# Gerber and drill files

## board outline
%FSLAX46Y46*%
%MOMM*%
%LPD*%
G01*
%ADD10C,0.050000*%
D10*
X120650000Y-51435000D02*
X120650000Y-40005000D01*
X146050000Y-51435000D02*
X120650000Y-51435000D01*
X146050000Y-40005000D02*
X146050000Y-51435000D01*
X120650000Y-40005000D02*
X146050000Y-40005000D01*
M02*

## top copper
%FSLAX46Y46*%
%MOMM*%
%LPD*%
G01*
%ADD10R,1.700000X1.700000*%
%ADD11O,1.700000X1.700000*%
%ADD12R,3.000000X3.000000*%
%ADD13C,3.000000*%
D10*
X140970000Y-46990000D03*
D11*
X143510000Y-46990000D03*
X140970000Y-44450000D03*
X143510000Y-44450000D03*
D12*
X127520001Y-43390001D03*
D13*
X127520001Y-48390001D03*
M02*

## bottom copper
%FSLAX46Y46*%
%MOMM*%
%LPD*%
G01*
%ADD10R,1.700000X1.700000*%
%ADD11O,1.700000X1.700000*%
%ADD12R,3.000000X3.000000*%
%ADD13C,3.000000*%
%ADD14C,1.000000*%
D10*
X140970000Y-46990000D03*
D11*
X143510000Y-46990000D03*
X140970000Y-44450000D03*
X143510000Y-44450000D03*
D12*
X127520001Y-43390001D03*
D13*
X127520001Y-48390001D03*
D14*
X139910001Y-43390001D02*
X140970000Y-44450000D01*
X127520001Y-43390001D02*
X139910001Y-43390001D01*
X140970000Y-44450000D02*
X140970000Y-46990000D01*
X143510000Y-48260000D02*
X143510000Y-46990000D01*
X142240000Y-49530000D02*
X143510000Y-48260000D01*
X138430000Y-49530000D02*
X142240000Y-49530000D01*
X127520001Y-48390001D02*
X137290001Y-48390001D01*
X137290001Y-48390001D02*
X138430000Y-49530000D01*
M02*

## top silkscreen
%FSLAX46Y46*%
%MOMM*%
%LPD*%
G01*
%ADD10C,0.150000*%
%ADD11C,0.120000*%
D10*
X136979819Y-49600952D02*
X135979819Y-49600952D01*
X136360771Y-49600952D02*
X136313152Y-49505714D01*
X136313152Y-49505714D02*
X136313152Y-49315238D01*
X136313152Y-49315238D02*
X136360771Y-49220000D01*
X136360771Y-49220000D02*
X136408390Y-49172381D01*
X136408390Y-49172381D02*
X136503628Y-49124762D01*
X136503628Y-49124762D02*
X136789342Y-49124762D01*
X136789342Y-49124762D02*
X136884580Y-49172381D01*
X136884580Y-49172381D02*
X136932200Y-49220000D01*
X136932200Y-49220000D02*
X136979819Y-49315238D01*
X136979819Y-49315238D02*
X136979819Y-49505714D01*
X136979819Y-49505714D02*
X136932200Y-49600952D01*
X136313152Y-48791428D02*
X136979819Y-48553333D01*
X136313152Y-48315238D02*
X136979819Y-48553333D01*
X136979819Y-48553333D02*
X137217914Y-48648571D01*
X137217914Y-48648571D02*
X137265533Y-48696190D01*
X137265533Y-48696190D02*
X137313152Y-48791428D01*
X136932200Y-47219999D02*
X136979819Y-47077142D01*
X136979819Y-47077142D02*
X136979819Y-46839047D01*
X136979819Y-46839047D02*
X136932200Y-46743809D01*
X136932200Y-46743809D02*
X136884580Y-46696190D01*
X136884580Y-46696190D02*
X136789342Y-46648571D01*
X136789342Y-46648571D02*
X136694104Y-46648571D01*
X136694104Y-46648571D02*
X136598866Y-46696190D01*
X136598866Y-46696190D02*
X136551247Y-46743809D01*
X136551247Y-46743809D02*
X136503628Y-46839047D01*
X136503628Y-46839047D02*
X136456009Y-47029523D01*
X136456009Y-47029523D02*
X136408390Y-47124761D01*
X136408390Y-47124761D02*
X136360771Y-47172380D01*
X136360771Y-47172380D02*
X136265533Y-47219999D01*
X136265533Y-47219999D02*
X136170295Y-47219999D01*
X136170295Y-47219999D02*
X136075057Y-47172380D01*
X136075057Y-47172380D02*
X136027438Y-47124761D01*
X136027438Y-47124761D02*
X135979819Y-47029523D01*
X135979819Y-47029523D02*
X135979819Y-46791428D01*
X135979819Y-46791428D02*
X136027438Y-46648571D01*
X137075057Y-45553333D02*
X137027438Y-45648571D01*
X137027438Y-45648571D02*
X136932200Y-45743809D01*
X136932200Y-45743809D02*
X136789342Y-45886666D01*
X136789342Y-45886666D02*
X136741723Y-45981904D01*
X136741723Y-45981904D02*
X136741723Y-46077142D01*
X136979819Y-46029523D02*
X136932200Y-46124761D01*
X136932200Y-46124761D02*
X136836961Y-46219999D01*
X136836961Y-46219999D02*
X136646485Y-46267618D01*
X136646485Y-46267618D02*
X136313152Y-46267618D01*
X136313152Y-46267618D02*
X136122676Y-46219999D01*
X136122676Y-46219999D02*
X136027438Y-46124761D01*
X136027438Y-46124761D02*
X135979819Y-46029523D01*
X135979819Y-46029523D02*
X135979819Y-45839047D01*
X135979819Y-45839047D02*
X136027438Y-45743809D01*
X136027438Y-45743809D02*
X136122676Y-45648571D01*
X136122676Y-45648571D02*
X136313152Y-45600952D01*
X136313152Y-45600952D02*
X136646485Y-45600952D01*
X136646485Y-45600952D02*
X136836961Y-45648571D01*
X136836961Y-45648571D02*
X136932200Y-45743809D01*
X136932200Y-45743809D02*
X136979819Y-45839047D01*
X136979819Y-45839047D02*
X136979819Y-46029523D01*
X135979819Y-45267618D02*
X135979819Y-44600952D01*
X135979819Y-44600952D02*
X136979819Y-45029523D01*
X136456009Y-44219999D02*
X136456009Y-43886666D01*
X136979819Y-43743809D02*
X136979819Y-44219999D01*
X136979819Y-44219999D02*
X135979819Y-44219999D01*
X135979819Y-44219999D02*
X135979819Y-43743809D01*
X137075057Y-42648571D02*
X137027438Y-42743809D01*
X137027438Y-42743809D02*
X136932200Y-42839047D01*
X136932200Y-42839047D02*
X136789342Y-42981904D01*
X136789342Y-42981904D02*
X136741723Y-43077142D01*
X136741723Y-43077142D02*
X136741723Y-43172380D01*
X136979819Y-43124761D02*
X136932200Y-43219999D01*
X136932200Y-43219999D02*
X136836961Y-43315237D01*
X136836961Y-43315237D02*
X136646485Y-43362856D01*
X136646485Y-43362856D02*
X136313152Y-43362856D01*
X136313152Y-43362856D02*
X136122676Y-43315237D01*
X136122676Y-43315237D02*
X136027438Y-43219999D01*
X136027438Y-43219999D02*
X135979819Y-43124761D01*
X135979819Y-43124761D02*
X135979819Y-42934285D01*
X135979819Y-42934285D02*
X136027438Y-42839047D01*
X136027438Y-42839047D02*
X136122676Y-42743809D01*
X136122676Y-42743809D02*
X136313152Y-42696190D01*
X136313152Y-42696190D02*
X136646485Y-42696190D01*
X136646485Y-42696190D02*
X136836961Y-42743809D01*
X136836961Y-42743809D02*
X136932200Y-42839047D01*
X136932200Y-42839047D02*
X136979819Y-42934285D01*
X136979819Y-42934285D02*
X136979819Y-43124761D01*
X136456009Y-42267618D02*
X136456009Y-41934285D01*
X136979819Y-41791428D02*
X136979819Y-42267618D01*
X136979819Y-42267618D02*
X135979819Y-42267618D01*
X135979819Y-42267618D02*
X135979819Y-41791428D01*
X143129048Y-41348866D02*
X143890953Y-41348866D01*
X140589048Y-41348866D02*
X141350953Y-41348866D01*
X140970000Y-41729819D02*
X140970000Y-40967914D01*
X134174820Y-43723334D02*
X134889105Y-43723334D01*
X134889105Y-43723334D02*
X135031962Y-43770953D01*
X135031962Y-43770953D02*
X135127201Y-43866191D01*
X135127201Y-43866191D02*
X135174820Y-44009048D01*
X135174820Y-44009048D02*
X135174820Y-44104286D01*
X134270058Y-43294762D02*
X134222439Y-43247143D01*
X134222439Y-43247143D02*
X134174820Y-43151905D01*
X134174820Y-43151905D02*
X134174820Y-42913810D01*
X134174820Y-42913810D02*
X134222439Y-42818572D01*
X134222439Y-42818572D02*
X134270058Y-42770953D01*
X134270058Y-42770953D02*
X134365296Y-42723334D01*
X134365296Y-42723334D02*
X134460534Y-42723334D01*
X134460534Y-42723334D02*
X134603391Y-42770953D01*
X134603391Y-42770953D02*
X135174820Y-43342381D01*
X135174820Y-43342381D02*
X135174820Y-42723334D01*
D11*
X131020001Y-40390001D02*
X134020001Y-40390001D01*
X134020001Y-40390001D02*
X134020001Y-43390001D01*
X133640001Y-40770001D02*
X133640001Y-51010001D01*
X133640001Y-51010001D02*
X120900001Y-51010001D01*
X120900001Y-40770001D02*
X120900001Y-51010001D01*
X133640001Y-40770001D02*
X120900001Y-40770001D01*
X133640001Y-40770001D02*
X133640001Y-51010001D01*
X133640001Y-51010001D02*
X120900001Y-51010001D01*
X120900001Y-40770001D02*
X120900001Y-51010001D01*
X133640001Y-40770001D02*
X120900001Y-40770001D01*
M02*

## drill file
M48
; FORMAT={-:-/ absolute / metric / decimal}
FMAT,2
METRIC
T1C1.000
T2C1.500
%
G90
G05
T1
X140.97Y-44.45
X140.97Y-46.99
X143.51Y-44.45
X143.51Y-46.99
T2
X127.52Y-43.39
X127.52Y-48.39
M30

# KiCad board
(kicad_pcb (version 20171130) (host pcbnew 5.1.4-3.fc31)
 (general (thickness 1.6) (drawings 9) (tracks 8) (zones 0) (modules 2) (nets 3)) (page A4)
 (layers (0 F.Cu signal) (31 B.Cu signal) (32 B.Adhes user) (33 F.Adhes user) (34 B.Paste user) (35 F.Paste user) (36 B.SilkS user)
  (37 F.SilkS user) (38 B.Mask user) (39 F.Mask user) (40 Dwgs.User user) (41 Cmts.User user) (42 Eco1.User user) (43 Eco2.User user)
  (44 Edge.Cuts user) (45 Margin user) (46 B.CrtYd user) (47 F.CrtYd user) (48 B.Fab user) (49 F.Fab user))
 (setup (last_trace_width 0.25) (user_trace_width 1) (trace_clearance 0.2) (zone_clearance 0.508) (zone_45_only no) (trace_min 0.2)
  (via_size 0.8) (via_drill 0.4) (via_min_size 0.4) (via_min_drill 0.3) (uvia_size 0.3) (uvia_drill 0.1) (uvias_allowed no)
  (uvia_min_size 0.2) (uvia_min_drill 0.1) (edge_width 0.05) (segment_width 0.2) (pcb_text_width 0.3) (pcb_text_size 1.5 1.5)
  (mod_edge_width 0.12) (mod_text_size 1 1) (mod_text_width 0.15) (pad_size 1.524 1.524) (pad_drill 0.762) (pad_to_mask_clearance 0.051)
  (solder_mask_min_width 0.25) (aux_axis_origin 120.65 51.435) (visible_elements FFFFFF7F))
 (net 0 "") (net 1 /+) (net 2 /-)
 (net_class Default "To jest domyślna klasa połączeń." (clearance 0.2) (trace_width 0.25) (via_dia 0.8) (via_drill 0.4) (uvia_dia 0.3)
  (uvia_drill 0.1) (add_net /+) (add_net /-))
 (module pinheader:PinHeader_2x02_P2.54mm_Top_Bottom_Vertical (layer B.Cu) (at 140.97 46.99)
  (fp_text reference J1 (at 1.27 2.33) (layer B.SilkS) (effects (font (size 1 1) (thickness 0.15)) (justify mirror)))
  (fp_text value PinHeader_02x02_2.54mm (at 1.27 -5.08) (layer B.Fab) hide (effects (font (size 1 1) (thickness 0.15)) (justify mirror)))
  (pad 1 thru_hole rect (at 0 0) (size 1.7 1.7) (drill 1) (layers *.Cu *.Mask) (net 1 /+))
  (pad 3 thru_hole oval (at 2.54 0) (size 1.7 1.7) (drill 1) (layers *.Cu *.Mask) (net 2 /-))
  (pad 2 thru_hole oval (at 0 -2.54) (size 1.7 1.7) (drill 1) (layers *.Cu *.Mask) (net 1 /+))
  (pad 4 thru_hole oval (at 2.54 -2.54) (size 1.7 1.7) (drill 1) (layers *.Cu *.Mask) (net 2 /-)))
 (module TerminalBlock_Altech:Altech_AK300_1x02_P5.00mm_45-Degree (layer F.Cu) (at 127.520001 43.390001 270)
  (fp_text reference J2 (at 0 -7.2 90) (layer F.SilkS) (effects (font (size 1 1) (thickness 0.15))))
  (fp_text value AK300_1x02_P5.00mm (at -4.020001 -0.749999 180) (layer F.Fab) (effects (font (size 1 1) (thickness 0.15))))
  (fp_line (start -3 -3.5) (end -3 -6.5) (layer F.SilkS) (width 0.12))
  (fp_line (start -3 -6.5) (end 0 -6.5) (layer F.SilkS) (width 0.12))
  (fp_line (start -2.62 -6.12) (end 7.62 -6.12) (layer F.SilkS) (width 0.12))
  (fp_line (start 7.62 -6.12) (end 7.62 6.62) (layer F.SilkS) (width 0.12))
  (fp_line (start -2.62 6.62) (end 7.62 6.62) (layer F.SilkS) (width 0.12))
  (fp_line (start -2.62 -6.12) (end -2.62 6.62) (layer F.SilkS) (width 0.12))
  (fp_line (start -2.62 -6.12) (end 7.62 -6.12) (layer F.SilkS) (width 0.12))
  (fp_line (start 7.62 -6.12) (end 7.62 6.62) (layer F.SilkS) (width 0.12))
  (fp_line (start -2.62 6.62) (end 7.62 6.62) (layer F.SilkS) (width 0.12))
  (fp_line (start -2.62 -6.12) (end -2.62 6.62) (layer F.SilkS) (width 0.12))
  (pad 1 thru_hole rect (at 0 0 270) (size 3 3) (drill 1.5) (layers *.Cu *.Mask) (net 1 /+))
  (pad 2 thru_hole circle (at 5 0 270) (size 3 3) (drill 1.5) (layers *.Cu *.Mask) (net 2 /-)))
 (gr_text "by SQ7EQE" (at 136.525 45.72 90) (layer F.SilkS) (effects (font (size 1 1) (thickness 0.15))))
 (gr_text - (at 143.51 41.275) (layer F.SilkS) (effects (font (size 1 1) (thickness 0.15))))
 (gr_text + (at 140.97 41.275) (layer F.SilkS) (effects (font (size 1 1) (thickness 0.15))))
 (gr_line (start 120.65 51.435) (end 120.65 40.005) (layer Edge.Cuts) (width 0.05))
 (gr_line (start 146.05 51.435) (end 120.65 51.435) (layer Edge.Cuts) (width 0.05))
 (gr_line (start 146.05 40.005) (end 146.05 51.435) (layer Edge.Cuts) (width 0.05))
 (gr_line (start 120.65 40.005) (end 146.05 40.005) (layer Edge.Cuts) (width 0.05))
 (segment (start 139.910001 43.390001) (end 140.97 44.45) (width 1) (layer B.Cu) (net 1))
 (segment (start 127.520001 43.390001) (end 139.910001 43.390001) (width 1) (layer B.Cu) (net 1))
 (segment (start 140.97 44.45) (end 140.97 46.99) (width 1) (layer B.Cu) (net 1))
 (segment (start 143.51 48.26) (end 143.51 46.99) (width 1) (layer B.Cu) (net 2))
 (segment (start 142.24 49.53) (end 143.51 48.26) (width 1) (layer B.Cu) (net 2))
 (segment (start 138.43 49.53) (end 142.24 49.53) (width 1) (layer B.Cu) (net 2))
 (segment (start 127.520001 48.390001) (end 137.290001 48.390001) (width 1) (layer B.Cu) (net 2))
 (segment (start 137.290001 48.390001) (end 138.43 49.53) (width 1) (layer B.Cu) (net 2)))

